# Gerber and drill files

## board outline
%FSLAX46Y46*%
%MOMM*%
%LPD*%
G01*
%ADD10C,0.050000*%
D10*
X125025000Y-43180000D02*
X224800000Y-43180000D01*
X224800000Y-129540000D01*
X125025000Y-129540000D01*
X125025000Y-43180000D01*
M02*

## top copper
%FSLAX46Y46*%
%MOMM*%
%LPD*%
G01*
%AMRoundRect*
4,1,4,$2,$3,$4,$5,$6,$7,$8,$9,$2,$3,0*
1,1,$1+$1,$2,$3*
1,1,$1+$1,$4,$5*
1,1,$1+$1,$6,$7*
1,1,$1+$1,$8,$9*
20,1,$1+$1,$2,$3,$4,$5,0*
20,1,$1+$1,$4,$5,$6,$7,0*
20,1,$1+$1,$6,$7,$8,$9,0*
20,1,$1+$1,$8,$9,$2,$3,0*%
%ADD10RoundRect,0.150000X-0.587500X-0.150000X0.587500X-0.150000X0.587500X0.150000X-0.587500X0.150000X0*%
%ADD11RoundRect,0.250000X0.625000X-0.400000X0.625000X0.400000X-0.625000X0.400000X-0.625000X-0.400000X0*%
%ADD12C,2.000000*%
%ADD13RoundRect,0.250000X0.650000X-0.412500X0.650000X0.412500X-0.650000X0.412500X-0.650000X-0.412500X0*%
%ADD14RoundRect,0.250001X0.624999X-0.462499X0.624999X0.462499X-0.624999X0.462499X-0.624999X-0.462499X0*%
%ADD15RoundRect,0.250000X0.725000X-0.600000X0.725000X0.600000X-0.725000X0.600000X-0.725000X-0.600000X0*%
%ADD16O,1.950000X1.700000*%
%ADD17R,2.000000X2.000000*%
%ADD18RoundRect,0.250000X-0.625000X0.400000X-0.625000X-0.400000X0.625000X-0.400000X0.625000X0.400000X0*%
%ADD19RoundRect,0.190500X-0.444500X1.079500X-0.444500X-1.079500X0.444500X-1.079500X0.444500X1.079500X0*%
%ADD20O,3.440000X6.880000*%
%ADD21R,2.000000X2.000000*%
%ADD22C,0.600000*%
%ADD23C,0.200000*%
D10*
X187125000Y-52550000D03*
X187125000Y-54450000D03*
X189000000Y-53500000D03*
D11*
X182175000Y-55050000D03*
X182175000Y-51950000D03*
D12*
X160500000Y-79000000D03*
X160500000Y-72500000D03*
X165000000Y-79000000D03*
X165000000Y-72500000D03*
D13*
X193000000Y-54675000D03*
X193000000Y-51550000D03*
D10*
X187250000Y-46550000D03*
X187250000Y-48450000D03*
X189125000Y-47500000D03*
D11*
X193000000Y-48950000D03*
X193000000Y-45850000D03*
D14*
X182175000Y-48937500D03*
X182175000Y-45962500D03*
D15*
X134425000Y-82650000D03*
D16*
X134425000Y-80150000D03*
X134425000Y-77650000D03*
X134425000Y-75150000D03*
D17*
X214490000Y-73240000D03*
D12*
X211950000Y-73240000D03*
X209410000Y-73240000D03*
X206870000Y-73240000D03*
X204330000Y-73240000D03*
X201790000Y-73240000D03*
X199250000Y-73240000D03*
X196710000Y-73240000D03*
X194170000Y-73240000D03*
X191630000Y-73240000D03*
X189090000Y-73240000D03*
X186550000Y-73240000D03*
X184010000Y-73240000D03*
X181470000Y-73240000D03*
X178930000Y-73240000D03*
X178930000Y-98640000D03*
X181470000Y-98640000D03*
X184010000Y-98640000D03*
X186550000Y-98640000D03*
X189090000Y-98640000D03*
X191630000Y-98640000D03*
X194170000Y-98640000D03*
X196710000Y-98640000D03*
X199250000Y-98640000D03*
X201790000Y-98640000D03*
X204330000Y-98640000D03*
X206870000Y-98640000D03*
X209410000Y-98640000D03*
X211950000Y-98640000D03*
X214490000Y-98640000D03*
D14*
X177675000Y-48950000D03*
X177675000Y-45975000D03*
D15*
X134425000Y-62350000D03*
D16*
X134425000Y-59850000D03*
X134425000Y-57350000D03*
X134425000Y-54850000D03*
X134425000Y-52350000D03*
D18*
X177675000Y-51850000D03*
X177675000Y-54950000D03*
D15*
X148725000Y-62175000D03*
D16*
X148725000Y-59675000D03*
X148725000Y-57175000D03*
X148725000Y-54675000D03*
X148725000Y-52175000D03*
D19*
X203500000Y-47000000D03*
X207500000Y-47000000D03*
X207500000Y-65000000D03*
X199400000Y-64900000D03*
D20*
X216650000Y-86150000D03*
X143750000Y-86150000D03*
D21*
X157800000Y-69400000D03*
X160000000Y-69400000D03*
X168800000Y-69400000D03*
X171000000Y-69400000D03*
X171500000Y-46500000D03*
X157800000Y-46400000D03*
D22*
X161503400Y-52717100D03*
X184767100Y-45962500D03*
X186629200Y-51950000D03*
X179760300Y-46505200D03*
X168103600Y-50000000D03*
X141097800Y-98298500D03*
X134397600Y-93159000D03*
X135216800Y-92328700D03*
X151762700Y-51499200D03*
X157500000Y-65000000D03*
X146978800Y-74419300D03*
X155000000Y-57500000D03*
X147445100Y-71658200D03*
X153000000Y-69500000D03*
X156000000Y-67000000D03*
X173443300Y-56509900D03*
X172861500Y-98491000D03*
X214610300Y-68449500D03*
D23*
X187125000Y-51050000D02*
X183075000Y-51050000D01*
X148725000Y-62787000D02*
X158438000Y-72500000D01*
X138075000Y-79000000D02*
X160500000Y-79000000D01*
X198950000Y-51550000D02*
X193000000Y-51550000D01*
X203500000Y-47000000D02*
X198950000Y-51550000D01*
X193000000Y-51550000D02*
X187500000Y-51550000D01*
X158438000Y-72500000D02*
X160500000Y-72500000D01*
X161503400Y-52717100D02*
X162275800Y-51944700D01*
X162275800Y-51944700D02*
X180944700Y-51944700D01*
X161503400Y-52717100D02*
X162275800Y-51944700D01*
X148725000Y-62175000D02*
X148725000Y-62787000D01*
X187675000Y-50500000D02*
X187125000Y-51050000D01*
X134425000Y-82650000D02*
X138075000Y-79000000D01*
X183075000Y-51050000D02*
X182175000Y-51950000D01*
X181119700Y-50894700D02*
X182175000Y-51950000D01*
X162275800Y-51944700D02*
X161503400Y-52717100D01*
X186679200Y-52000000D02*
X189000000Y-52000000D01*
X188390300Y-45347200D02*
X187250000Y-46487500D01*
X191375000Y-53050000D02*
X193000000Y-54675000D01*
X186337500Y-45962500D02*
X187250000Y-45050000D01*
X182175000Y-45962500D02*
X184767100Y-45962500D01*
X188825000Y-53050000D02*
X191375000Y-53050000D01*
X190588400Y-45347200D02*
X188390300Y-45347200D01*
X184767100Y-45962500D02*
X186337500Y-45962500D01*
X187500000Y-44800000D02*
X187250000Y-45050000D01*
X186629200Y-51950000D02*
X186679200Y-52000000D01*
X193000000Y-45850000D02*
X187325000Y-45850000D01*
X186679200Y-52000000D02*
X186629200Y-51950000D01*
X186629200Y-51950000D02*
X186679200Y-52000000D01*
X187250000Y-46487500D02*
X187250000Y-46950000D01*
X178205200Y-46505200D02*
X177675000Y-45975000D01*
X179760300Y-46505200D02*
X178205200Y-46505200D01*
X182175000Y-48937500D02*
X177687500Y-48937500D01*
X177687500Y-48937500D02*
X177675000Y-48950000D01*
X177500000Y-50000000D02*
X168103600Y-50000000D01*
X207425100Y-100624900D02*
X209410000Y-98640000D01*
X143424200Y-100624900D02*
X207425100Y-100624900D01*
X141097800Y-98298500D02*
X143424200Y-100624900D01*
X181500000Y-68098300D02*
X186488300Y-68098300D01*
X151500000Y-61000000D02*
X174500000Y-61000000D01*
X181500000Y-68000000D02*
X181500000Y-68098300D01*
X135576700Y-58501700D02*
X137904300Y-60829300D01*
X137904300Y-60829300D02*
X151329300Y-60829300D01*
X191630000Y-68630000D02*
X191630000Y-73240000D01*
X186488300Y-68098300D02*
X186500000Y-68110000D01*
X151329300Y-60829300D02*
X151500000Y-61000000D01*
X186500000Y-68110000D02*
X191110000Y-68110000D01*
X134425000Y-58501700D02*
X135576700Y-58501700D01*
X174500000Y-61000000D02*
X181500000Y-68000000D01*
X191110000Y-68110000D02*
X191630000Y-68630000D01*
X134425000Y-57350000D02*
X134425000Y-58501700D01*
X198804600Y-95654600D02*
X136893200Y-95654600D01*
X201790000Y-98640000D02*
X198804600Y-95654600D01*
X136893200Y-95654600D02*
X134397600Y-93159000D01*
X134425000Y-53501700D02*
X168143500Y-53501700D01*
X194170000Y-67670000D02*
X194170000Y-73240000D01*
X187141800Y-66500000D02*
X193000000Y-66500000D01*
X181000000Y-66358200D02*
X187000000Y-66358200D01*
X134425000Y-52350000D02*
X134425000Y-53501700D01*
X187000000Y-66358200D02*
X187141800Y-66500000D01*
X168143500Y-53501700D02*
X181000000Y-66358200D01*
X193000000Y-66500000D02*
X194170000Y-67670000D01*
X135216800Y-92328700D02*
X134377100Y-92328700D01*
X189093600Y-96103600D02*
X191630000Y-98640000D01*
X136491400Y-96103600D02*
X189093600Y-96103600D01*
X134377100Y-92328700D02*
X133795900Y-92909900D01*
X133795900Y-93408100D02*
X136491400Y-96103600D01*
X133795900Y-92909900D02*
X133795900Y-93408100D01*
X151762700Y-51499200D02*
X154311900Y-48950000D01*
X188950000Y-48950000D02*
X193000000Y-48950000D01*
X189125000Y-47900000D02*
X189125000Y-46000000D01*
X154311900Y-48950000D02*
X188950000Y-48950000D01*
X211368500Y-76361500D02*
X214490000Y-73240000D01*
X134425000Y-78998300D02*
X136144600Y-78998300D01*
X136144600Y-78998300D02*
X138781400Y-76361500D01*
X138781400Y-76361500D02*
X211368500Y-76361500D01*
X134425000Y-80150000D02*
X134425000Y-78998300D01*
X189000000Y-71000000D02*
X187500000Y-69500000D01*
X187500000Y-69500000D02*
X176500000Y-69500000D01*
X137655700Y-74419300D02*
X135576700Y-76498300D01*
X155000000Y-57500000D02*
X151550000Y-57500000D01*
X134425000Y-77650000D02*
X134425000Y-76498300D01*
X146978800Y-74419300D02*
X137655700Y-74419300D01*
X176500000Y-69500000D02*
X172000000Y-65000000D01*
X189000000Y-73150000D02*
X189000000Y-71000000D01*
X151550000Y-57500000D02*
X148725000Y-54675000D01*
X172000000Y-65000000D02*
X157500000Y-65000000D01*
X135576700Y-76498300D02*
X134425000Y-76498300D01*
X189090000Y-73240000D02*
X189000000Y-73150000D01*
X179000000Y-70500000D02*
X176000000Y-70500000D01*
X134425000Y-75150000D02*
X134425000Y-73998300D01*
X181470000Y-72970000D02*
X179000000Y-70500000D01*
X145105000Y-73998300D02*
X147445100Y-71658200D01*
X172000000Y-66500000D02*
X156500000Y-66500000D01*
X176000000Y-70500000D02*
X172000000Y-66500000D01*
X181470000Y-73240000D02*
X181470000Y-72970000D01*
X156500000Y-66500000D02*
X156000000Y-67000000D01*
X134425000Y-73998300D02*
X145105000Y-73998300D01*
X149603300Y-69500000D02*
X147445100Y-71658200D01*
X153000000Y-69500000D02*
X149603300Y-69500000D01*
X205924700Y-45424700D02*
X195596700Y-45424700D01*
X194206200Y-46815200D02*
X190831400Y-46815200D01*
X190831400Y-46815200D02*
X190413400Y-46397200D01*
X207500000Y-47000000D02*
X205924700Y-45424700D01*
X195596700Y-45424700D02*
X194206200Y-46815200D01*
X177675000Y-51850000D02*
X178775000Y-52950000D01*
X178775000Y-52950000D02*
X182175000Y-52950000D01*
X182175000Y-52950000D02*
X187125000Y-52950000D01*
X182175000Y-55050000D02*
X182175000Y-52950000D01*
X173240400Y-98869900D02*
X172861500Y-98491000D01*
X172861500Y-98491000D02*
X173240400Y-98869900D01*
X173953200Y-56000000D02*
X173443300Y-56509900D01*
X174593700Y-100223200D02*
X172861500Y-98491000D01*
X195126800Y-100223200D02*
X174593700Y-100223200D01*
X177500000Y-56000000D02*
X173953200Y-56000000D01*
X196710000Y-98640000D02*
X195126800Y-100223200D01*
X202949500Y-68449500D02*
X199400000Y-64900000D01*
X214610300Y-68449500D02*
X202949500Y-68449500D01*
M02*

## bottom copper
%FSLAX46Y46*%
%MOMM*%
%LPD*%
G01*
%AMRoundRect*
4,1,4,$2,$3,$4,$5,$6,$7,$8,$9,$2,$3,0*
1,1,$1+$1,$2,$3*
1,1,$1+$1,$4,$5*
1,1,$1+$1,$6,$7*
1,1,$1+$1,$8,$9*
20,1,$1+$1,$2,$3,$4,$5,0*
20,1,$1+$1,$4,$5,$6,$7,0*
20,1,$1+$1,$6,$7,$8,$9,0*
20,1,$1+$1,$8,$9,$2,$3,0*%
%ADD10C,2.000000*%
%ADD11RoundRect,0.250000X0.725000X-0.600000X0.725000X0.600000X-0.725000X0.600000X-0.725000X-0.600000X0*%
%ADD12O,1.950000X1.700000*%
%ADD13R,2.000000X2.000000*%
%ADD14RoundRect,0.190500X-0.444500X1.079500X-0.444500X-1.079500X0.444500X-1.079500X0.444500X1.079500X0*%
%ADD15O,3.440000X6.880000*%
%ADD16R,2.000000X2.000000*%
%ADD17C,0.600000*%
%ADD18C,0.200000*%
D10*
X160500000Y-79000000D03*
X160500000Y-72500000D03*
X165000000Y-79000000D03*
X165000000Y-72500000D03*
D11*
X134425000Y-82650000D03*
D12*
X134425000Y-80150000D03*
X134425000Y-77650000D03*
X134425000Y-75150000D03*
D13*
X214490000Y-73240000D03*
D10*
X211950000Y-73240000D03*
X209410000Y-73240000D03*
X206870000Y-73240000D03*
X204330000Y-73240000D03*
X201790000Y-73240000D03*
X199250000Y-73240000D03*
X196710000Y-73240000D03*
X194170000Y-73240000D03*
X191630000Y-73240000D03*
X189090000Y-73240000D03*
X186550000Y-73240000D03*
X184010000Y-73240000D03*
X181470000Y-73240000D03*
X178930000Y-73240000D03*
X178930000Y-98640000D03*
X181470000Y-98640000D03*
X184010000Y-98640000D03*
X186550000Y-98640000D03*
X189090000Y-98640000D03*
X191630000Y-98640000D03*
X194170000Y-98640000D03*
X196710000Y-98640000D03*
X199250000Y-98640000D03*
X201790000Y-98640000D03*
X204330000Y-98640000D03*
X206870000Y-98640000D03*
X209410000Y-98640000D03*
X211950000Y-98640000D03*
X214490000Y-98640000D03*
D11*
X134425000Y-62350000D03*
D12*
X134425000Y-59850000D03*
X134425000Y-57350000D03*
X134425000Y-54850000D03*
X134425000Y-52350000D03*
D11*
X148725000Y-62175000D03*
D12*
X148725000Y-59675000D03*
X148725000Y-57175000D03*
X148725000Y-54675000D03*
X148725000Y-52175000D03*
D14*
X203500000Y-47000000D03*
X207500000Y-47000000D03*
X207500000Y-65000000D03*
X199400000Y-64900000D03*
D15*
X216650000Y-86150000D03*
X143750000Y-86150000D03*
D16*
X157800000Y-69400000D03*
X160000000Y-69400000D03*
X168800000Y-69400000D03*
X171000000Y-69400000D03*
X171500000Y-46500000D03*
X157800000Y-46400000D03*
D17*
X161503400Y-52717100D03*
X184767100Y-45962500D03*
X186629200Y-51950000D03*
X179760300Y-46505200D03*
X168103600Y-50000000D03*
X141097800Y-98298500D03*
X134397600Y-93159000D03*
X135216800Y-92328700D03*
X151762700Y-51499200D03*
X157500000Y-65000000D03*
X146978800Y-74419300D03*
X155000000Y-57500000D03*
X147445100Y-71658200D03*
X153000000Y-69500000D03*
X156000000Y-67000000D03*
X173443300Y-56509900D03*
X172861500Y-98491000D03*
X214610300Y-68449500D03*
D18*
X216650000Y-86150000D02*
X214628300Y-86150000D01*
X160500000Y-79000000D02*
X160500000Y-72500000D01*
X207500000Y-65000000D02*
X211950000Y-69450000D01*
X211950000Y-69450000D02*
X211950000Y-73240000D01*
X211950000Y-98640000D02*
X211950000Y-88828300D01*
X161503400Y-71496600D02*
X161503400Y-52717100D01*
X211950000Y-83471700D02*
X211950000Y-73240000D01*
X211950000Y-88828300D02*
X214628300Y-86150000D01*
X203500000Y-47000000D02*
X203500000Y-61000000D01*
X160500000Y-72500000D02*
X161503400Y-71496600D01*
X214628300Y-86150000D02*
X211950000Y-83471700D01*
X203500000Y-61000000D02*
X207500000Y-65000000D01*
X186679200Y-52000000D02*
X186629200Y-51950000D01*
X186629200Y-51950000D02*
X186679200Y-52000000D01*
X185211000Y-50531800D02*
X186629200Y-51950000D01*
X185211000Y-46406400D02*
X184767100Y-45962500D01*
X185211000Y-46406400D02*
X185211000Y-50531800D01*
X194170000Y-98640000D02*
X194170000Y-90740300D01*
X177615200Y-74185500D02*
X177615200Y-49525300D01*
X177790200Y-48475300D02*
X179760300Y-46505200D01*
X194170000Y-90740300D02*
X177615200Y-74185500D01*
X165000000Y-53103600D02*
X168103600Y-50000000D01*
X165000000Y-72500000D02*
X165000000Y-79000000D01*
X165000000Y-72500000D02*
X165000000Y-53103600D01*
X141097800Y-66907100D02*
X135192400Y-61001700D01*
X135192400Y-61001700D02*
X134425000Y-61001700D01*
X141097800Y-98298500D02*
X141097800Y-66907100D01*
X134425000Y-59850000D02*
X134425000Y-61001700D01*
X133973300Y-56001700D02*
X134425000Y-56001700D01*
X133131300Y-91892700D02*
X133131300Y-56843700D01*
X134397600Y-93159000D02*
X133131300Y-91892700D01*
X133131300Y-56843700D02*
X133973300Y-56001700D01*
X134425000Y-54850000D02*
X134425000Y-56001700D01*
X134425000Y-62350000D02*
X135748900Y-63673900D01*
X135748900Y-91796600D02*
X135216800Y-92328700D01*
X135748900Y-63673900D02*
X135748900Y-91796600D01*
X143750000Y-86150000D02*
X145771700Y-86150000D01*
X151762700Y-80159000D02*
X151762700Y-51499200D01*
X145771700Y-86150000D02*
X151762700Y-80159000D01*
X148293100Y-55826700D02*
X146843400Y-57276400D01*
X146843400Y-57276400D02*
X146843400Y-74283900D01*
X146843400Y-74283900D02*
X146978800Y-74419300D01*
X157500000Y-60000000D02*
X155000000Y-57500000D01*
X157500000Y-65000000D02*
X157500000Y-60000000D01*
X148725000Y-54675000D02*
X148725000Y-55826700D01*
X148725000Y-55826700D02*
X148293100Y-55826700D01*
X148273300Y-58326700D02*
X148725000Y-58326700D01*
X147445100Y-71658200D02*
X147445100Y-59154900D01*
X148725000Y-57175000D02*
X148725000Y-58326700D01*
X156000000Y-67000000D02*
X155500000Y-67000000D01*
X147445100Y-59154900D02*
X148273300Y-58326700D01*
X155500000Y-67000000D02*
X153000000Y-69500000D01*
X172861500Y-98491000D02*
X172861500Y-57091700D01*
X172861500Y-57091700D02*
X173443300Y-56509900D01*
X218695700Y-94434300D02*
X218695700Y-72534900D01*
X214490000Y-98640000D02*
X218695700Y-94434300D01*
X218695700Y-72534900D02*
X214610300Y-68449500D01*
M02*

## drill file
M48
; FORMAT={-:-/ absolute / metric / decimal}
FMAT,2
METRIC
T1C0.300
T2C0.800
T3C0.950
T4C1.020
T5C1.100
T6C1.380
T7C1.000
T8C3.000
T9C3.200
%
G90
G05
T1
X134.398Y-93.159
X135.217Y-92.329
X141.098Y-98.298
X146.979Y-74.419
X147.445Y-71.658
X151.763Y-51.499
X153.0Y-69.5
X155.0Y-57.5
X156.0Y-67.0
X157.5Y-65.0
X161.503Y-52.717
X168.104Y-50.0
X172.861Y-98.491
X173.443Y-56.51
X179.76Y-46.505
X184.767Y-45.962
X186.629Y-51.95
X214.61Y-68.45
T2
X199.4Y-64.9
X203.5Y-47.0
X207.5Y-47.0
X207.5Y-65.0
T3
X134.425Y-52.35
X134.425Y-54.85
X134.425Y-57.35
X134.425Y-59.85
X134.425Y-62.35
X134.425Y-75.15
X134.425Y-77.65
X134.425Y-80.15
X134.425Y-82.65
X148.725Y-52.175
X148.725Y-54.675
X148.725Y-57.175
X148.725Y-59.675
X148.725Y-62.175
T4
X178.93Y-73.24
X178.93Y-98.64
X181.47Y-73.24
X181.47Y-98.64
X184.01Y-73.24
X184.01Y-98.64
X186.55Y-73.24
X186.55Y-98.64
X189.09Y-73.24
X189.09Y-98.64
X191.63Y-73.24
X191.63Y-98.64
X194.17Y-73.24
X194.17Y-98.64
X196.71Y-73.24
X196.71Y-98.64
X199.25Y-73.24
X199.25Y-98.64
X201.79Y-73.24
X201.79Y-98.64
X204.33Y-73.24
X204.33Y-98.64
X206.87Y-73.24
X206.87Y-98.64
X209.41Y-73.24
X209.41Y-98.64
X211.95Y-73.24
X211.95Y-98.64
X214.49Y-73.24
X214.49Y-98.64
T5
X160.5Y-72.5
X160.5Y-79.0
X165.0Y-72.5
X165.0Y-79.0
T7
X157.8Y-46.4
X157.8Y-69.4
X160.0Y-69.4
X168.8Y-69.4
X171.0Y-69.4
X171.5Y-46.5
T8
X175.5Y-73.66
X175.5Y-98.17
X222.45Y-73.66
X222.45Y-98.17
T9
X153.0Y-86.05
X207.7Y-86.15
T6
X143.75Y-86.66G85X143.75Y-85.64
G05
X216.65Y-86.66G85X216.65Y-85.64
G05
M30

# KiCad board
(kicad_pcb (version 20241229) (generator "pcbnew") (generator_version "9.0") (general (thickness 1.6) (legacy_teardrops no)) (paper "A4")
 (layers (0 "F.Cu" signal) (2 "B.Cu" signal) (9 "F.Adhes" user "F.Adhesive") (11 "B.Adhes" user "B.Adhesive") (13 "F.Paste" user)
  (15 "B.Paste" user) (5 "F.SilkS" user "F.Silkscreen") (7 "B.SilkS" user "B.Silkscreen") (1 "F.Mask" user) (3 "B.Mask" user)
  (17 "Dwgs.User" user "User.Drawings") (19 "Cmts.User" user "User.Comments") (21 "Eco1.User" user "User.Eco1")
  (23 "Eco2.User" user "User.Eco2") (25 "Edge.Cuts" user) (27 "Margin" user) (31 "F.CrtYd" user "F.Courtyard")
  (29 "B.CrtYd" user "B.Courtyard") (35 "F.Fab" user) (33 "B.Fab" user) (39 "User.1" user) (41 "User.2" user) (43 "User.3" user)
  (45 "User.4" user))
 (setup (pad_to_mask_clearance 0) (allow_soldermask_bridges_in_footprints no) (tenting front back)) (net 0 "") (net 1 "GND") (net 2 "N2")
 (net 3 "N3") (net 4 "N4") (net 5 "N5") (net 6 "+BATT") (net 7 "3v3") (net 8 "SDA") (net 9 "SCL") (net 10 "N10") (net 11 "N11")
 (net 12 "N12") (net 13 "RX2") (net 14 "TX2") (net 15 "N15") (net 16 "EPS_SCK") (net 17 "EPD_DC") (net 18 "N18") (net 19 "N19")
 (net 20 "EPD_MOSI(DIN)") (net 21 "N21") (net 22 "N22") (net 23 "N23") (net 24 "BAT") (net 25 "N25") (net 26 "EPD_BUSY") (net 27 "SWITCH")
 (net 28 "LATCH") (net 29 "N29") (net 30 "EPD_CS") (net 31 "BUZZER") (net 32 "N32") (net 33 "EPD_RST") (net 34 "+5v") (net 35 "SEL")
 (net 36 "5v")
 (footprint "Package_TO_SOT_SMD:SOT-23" (layer "F.Cu") (at 188.0625 53.5)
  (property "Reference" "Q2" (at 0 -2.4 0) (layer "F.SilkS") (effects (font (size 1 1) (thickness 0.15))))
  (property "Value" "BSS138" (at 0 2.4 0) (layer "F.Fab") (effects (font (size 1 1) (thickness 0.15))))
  (pad "1" smd roundrect (at -0.9375 -0.95) (size 1.475 0.6) (layers "F.Cu" "F.Mask" "F.Paste") (roundrect_rratio 0.25) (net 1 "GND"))
  (pad "2" smd roundrect (at -0.9375 0.95) (size 1.475 0.6) (layers "F.Cu" "F.Mask" "F.Paste") (roundrect_rratio 0.25) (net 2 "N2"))
  (pad "3" smd roundrect (at 0.9375 0) (size 1.475 0.6) (layers "F.Cu" "F.Mask" "F.Paste") (roundrect_rratio 0.25) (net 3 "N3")))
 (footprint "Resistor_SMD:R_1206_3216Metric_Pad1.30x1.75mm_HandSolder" (layer "F.Cu") (at 182.175 53.5 90)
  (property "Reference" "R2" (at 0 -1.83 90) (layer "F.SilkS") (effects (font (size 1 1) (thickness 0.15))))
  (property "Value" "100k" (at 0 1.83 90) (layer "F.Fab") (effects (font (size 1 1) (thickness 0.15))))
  (pad "1" smd roundrect (at -1.55 0 90) (size 1.3 1.75) (layers "F.Cu" "F.Mask" "F.Paste") (roundrect_rratio 0.192308) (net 2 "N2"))
  (pad "2" smd roundrect (at 1.55 0 90) (size 1.3 1.75) (layers "F.Cu" "F.Mask" "F.Paste") (roundrect_rratio 0.192308) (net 1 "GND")))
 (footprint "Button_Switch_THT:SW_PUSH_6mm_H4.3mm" (layer "F.Cu") (at 160.5 79 90)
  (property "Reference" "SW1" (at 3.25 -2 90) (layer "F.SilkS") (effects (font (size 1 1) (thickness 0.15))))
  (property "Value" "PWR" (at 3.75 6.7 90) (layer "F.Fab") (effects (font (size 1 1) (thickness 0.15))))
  (pad "1" thru_hole circle (at 0 0 180) (size 2 2) (drill 1.1) (layers "*.Cu" "*.Mask") (remove_unused_layers no) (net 1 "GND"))
  (pad "1" thru_hole circle (at 6.5 0 180) (size 2 2) (drill 1.1) (layers "*.Cu" "*.Mask") (remove_unused_layers no) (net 1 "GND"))
  (pad "2" thru_hole circle (at 0 4.5 180) (size 2 2) (drill 1.1) (layers "*.Cu" "*.Mask") (remove_unused_layers no) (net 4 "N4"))
  (pad "2" thru_hole circle (at 6.5 4.5 180) (size 2 2) (drill 1.1) (layers "*.Cu" "*.Mask") (remove_unused_layers no) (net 4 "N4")))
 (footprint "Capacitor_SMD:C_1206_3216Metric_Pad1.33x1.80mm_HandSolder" (layer "F.Cu") (at 193 53.1125 90)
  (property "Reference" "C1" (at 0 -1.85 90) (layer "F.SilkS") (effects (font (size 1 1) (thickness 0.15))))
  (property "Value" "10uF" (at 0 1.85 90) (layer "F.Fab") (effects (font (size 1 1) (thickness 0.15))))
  (pad "1" smd roundrect (at -1.5625 0 90) (size 1.325 1.8) (layers "F.Cu" "F.Mask" "F.Paste") (roundrect_rratio 0.188679) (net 3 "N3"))
  (pad "2" smd roundrect (at 1.5625 0 90) (size 1.325 1.8) (layers "F.Cu" "F.Mask" "F.Paste") (roundrect_rratio 0.188679) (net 1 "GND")))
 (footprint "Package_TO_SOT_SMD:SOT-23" (layer "F.Cu") (at 188.1875 47.5)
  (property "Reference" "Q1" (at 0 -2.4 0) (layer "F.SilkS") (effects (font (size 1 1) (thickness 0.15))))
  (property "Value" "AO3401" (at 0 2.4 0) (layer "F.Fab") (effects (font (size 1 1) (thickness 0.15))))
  (pad "1" smd roundrect (at -0.9375 -0.95) (size 1.475 0.6) (layers "F.Cu" "F.Mask" "F.Paste") (roundrect_rratio 0.25) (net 3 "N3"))
  (pad "2" smd roundrect (at -0.9375 0.95) (size 1.475 0.6) (layers "F.Cu" "F.Mask" "F.Paste") (roundrect_rratio 0.25) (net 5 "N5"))
  (pad "3" smd roundrect (at 0.9375 0) (size 1.475 0.6) (layers "F.Cu" "F.Mask" "F.Paste") (roundrect_rratio 0.25) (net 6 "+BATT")))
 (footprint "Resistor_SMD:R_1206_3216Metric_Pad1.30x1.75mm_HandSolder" (layer "F.Cu") (at 193 47.4 90)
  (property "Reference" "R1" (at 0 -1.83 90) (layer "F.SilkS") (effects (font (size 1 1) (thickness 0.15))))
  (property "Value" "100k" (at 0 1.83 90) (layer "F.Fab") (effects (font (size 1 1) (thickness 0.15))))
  (pad "1" smd roundrect (at -1.55 0 90) (size 1.3 1.75) (layers "F.Cu" "F.Mask" "F.Paste") (roundrect_rratio 0.192308) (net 6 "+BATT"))
  (pad "2" smd roundrect (at 1.55 0 90) (size 1.3 1.75) (layers "F.Cu" "F.Mask" "F.Paste") (roundrect_rratio 0.192308) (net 3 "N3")))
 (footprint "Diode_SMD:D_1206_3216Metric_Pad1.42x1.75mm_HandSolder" (layer "F.Cu") (at 182.175 47.45 90)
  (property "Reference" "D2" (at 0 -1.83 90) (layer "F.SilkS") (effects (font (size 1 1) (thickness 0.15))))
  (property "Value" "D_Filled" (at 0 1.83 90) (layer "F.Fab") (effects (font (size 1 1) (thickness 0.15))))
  (pad "1" smd roundrect (at -1.4875 0 90) (size 1.425 1.75) (layers "F.Cu" "F.Mask" "F.Paste") (roundrect_rratio 0.175439) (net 4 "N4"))
  (pad "2" smd roundrect (at 1.4875 0 90) (size 1.425 1.75) (layers "F.Cu" "F.Mask" "F.Paste") (roundrect_rratio 0.175439) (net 3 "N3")))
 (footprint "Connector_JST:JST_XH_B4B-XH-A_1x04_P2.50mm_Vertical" (layer "F.Cu") (at 134.425 82.65 90)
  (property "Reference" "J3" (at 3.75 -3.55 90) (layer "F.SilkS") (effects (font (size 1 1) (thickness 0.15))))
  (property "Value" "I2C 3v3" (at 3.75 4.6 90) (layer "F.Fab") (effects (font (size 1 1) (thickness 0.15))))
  (pad "1" thru_hole roundrect (at 0 0 90) (size 1.7 1.95) (drill 0.95) (layers "*.Cu" "*.Mask") (remove_unused_layers no)
   (roundrect_rratio 0.147059) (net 1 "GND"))
  (pad "2" thru_hole oval (at 2.5 0 90) (size 1.7 1.95) (drill 0.95) (layers "*.Cu" "*.Mask") (remove_unused_layers no) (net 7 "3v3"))
  (pad "3" thru_hole oval (at 5 0 90) (size 1.7 1.95) (drill 0.95) (layers "*.Cu" "*.Mask") (remove_unused_layers no) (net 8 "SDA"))
  (pad "4" thru_hole oval (at 7.5 0 90) (size 1.7 1.95) (drill 0.95) (layers "*.Cu" "*.Mask") (remove_unused_layers no) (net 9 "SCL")))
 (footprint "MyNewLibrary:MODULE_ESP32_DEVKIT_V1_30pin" (layer "F.Cu") (at 198.975 85.94 -90)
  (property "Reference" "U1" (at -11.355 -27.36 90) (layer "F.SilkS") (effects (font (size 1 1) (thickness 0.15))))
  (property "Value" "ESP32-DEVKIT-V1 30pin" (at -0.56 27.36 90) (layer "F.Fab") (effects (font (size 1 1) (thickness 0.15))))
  (pad "" np_thru_hole circle (at -12.28 -23.475 270) (size 3 3) (drill 3) (layers "*.Cu" "*.Mask"))
  (pad "" np_thru_hole circle (at -12.28 23.475 270) (size 3 3) (drill 3) (layers "*.Cu" "*.Mask"))
  (pad "" np_thru_hole circle (at 12.23 -23.475 270) (size 3 3) (drill 3) (layers "*.Cu" "*.Mask"))
  (pad "" np_thru_hole circle (at 12.23 23.475 270) (size 3 3) (drill 3) (layers "*.Cu" "*.Mask"))
  (pad "1" thru_hole rect (at -12.7 -15.515 270) (size 2 2) (drill 1.02) (layers "*.Cu" "*.Mask") (remove_unused_layers no) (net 7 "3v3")
   (solder_mask_margin 0.102))
  (pad "2" thru_hole circle (at -12.7 -12.975 270) (size 2 2) (drill 1.02) (layers "*.Cu" "*.Mask") (remove_unused_layers no) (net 1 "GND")
   (solder_mask_margin 0.102))
  (pad "3" thru_hole circle (at -12.7 -10.435 270) (size 2 2) (drill 1.02) (layers "*.Cu" "*.Mask") (remove_unused_layers no) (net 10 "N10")
   (solder_mask_margin 0.102))
  (pad "4" thru_hole circle (at -12.7 -7.895 270) (size 2 2) (drill 1.02) (layers "*.Cu" "*.Mask") (remove_unused_layers no) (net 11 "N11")
   (solder_mask_margin 0.102))
  (pad "5" thru_hole circle (at -12.7 -5.355 270) (size 2 2) (drill 1.02) (layers "*.Cu" "*.Mask") (remove_unused_layers no) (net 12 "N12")
   (solder_mask_margin 0.102))
  (pad "6" thru_hole circle (at -12.7 -2.815 270) (size 2 2) (drill 1.02) (layers "*.Cu" "*.Mask") (remove_unused_layers no) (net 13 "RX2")
   (solder_mask_margin 0.102))
  (pad "7" thru_hole circle (at -12.7 -0.275 270) (size 2 2) (drill 1.02) (layers "*.Cu" "*.Mask") (remove_unused_layers no) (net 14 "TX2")
   (solder_mask_margin 0.102))
  (pad "8" thru_hole circle (at -12.7 2.265 270) (size 2 2) (drill 1.02) (layers "*.Cu" "*.Mask") (remove_unused_layers no) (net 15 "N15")
   (solder_mask_margin 0.102))
  (pad "9" thru_hole circle (at -12.7 4.805 270) (size 2 2) (drill 1.02) (layers "*.Cu" "*.Mask") (remove_unused_layers no)
   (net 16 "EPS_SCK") (solder_mask_margin 0.102))
  (pad "10" thru_hole circle (at -12.7 7.345 270) (size 2 2) (drill 1.02) (layers "*.Cu" "*.Mask") (remove_unused_layers no)
   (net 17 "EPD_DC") (solder_mask_margin 0.102))
  (pad "11" thru_hole circle (at -12.7 9.885 270) (size 2 2) (drill 1.02) (layers "*.Cu" "*.Mask") (remove_unused_layers no) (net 8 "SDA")
   (solder_mask_margin 0.102))
  (pad "12" thru_hole circle (at -12.7 12.425 270) (size 2 2) (drill 1.02) (layers "*.Cu" "*.Mask") (remove_unused_layers no) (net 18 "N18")
   (solder_mask_margin 0.102))
  (pad "13" thru_hole circle (at -12.7 14.965 270) (size 2 2) (drill 1.02) (layers "*.Cu" "*.Mask") (remove_unused_layers no) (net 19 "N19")
   (solder_mask_margin 0.102))
  (pad "14" thru_hole circle (at -12.7 17.505 270) (size 2 2) (drill 1.02) (layers "*.Cu" "*.Mask") (remove_unused_layers no) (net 9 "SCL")
   (solder_mask_margin 0.102))
  (pad "15" thru_hole circle (at -12.7 20.045 270) (size 2 2) (drill 1.02) (layers "*.Cu" "*.Mask") (remove_unused_layers no)
   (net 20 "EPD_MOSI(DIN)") (solder_mask_margin 0.102))
  (pad "16" thru_hole circle (at 12.7 20.045 270) (size 2 2) (drill 1.02) (layers "*.Cu" "*.Mask") (remove_unused_layers no) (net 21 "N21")
   (solder_mask_margin 0.102))
  (pad "17" thru_hole circle (at 12.7 17.505 270) (size 2 2) (drill 1.02) (layers "*.Cu" "*.Mask") (remove_unused_layers no) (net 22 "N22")
   (solder_mask_margin 0.102))
  (pad "18" thru_hole circle (at 12.7 14.965 270) (size 2 2) (drill 1.02) (layers "*.Cu" "*.Mask") (remove_unused_layers no) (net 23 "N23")
   (solder_mask_margin 0.102))
  (pad "19" thru_hole circle (at 12.7 12.425 270) (size 2 2) (drill 1.02) (layers "*.Cu" "*.Mask") (remove_unused_layers no) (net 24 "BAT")
   (solder_mask_margin 0.102))
  (pad "20" thru_hole circle (at 12.7 9.885 270) (size 2 2) (drill 1.02) (layers "*.Cu" "*.Mask") (remove_unused_layers no) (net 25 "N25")
   (solder_mask_margin 0.102))
  (pad "21" thru_hole circle (at 12.7 7.345 270) (size 2 2) (drill 1.02) (layers "*.Cu" "*.Mask") (remove_unused_layers no)
   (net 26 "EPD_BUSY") (solder_mask_margin 0.102))
  (pad "22" thru_hole circle (at 12.7 4.805 270) (size 2 2) (drill 1.02) (layers "*.Cu" "*.Mask") (remove_unused_layers no)
   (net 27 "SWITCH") (solder_mask_margin 0.102))
  (pad "23" thru_hole circle (at 12.7 2.265 270) (size 2 2) (drill 1.02) (layers "*.Cu" "*.Mask") (remove_unused_layers no) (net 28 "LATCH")
   (solder_mask_margin 0.102))
  (pad "24" thru_hole circle (at 12.7 -0.275 270) (size 2 2) (drill 1.02) (layers "*.Cu" "*.Mask") (remove_unused_layers no) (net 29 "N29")
   (solder_mask_margin 0.102))
  (pad "25" thru_hole circle (at 12.7 -2.815 270) (size 2 2) (drill 1.02) (layers "*.Cu" "*.Mask") (remove_unused_layers no)
   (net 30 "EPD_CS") (solder_mask_margin 0.102))
  (pad "26" thru_hole circle (at 12.7 -5.355 270) (size 2 2) (drill 1.02) (layers "*.Cu" "*.Mask") (remove_unused_layers no)
   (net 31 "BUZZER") (solder_mask_margin 0.102))
  (pad "27" thru_hole circle (at 12.7 -7.895 270) (size 2 2) (drill 1.02) (layers "*.Cu" "*.Mask") (remove_unused_layers no) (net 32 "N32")
   (solder_mask_margin 0.102))
  (pad "28" thru_hole circle (at 12.7 -10.435 270) (size 2 2) (drill 1.02) (layers "*.Cu" "*.Mask") (remove_unused_layers no)
   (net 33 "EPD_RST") (solder_mask_margin 0.102))
  (pad "29" thru_hole circle (at 12.7 -12.975 270) (size 2 2) (drill 1.02) (layers "*.Cu" "*.Mask") (remove_unused_layers no) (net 1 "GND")
   (solder_mask_margin 0.102))
  (pad "30" thru_hole circle (at 12.7 -15.515 270) (size 2 2) (drill 1.02) (layers "*.Cu" "*.Mask") (remove_unused_layers no) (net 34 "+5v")
   (solder_mask_margin 0.102))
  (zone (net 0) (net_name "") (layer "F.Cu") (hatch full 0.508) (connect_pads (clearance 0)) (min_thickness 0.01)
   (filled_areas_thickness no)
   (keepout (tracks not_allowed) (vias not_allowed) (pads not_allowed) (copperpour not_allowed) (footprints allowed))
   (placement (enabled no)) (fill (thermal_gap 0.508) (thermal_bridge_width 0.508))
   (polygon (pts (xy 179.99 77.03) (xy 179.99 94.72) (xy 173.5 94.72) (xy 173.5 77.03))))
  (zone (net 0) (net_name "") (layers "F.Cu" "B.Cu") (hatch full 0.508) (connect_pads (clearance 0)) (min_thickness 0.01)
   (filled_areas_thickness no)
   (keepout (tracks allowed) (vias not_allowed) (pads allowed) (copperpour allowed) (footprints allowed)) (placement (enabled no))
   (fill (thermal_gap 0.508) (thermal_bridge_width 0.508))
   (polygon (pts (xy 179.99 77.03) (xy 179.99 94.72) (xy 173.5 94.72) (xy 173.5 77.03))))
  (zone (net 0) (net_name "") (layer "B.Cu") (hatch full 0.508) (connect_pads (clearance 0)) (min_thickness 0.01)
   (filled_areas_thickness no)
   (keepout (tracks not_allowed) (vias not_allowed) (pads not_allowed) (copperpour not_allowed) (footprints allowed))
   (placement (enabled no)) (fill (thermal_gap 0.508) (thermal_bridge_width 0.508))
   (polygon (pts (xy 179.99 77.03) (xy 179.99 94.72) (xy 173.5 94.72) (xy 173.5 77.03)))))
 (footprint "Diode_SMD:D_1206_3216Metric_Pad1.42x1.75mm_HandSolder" (layer "F.Cu") (at 177.675 47.4625 90)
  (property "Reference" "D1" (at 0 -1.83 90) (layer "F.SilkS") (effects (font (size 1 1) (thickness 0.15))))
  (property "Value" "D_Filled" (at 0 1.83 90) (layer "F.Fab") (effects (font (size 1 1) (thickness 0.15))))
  (pad "1" smd roundrect (at -1.4875 0 90) (size 1.425 1.75) (layers "F.Cu" "F.Mask" "F.Paste") (roundrect_rratio 0.175439) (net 4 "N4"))
  (pad "2" smd roundrect (at 1.4875 0 90) (size 1.425 1.75) (layers "F.Cu" "F.Mask" "F.Paste") (roundrect_rratio 0.175439) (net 27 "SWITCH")))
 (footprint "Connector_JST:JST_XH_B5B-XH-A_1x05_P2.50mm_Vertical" (layer "F.Cu") (at 134.425 62.35 90)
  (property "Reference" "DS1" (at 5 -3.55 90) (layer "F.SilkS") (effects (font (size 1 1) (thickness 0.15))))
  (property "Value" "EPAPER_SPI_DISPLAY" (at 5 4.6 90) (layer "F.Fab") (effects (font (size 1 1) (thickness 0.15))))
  (pad "1" thru_hole roundrect (at 0 0 90) (size 1.7 1.95) (drill 0.95) (layers "*.Cu" "*.Mask") (remove_unused_layers no)
   (roundrect_rratio 0.147059) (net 26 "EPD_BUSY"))
  (pad "2" thru_hole oval (at 2.5 0 90) (size 1.7 1.95) (drill 0.95) (layers "*.Cu" "*.Mask") (remove_unused_layers no) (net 33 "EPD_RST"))
  (pad "3" thru_hole oval (at 5 0 90) (size 1.7 1.95) (drill 0.95) (layers "*.Cu" "*.Mask") (remove_unused_layers no) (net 17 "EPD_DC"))
  (pad "4" thru_hole oval (at 7.5 0 90) (size 1.7 1.95) (drill 0.95) (layers "*.Cu" "*.Mask") (remove_unused_layers no) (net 30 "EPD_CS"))
  (pad "5" thru_hole oval (at 10 0 90) (size 1.7 1.95) (drill 0.95) (layers "*.Cu" "*.Mask") (remove_unused_layers no) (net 16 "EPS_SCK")))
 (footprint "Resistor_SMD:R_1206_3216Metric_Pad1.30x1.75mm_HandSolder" (layer "F.Cu") (at 177.675 53.4 -90)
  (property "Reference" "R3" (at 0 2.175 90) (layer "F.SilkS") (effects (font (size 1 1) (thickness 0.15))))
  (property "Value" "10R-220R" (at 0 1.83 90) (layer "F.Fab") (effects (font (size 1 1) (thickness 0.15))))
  (pad "1" smd roundrect (at -1.55 0 270) (size 1.3 1.75) (layers "F.Cu" "F.Mask" "F.Paste") (roundrect_rratio 0.192308) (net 2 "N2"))
  (pad "2" smd roundrect (at 1.55 0 270) (size 1.3 1.75) (layers "F.Cu" "F.Mask" "F.Paste") (roundrect_rratio 0.192308) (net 28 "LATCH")))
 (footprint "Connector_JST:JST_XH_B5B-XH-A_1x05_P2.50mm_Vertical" (layer "F.Cu") (at 148.725 62.175 90)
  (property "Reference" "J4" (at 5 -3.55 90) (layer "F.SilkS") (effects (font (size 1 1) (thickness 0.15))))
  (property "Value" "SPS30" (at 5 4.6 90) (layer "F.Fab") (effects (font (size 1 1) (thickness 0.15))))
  (pad "1" thru_hole roundrect (at 0 0 90) (size 1.7 1.95) (drill 0.95) (layers "*.Cu" "*.Mask") (remove_unused_layers no)
   (roundrect_rratio 0.147059) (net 1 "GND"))
  (pad "2" thru_hole oval (at 2.5 0 90) (size 1.7 1.95) (drill 0.95) (layers "*.Cu" "*.Mask") (remove_unused_layers no) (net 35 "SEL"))
  (pad "3" thru_hole oval (at 5 0 90) (size 1.7 1.95) (drill 0.95) (layers "*.Cu" "*.Mask") (remove_unused_layers no) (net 9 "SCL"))
  (pad "4" thru_hole oval (at 7.5 0 90) (size 1.7 1.95) (drill 0.95) (layers "*.Cu" "*.Mask") (remove_unused_layers no) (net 8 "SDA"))
  (pad "5" thru_hole oval (at 10 0 90) (size 1.7 1.95) (drill 0.95) (layers "*.Cu" "*.Mask") (remove_unused_layers no) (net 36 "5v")))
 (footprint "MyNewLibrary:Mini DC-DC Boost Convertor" (layer "B.Cu") (at 203.4 56.1 -90)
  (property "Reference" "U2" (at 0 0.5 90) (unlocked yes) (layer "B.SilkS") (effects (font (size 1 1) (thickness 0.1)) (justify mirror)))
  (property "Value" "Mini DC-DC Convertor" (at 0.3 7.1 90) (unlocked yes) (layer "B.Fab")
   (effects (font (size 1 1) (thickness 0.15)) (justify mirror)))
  (pad "1" thru_hole roundrect (at -9.1 -0.1 270) (size 2.54 1.27) (drill 0.8) (layers "*.Cu" "*.Mask") (remove_unused_layers no)
   (roundrect_rratio 0.15) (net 1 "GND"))
  (pad "2" thru_hole roundrect (at -9.1 -4.1 270) (size 2.54 1.27) (drill 0.8) (layers "*.Cu" "*.Mask") (remove_unused_layers no)
   (roundrect_rratio 0.15) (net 5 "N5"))
  (pad "3" thru_hole roundrect (at 8.9 -4.1 270) (size 2.54 1.27) (drill 0.8) (layers "*.Cu" "*.Mask") (remove_unused_layers no)
   (roundrect_rratio 0.15) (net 1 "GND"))
  (pad "4" thru_hole roundrect (at 8.8 4 270) (size 2.54 1.27) (drill 0.8) (layers "*.Cu" "*.Mask") (remove_unused_layers no)
   (roundrect_rratio 0.15) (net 34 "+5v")))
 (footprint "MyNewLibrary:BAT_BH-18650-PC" (layer "B.Cu") (at 180.2 86.15 180)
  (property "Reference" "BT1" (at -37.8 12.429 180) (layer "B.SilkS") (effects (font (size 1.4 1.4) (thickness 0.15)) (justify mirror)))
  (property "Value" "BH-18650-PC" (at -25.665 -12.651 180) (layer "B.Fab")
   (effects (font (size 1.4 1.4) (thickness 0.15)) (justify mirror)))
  (pad "" np_thru_hole circle (at -27.5 0 180) (size 3.2 3.2) (drill 3.2) (layers "*.Cu" "*.Mask"))
  (pad "" np_thru_hole circle (at 27.2 0.1 180) (size 3.2 3.2) (drill 3.2) (layers "*.Cu" "*.Mask"))
  (pad "N" thru_hole oval (at -36.45 0 180) (size 3.44 6.88) (drill oval 1.38 2.4) (layers "*.Cu" "*.Mask") (remove_unused_layers no)
   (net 1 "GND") (solder_mask_margin 0.102))
  (pad "P" thru_hole oval (at 36.45 0 180) (size 3.44 6.88) (drill oval 1.38 2.4) (layers "*.Cu" "*.Mask") (remove_unused_layers no)
   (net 6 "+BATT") (solder_mask_margin 0.102)))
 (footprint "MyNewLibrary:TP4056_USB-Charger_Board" (layer "B.Cu") (at 164.3 57 90)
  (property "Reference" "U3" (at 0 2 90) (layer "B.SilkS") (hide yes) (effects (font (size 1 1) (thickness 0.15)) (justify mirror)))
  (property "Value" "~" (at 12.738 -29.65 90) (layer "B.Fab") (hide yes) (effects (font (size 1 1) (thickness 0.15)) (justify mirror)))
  (pad "" np_thru_hole rect (at -12.4 -6.5 90) (size 2 2) (drill 1) (layers "*.Cu" "*.Mask"))
  (pad "" np_thru_hole rect (at -12.4 -4.3 90) (size 2 2) (drill 1) (layers "*.Cu" "*.Mask"))
  (pad "" np_thru_hole rect (at -12.4 4.5 90) (size 2 2) (drill 1) (layers "*.Cu" "*.Mask"))
  (pad "" np_thru_hole rect (at -12.4 6.7 90) (size 2 2) (drill 1) (layers "*.Cu" "*.Mask"))
  (pad "" np_thru_hole rect (at 10.5 7.2 90) (size 2 2) (drill 1) (layers "*.Cu" "*.Mask"))
  (pad "" np_thru_hole rect (at 10.6 -6.5 90) (size 2 2) (drill 1) (layers "*.Cu" "*.Mask")))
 (gr_rect (start 125.025 43.18) (end 224.8 129.54) (stroke (width 0.05) (type default)) (fill no) (layer "Edge.Cuts"))
 (segment (start 187.125 51.05) (end 183.075 51.05) (width 0.2) (layer "F.Cu") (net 1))
 (segment (start 148.725 62.787) (end 158.438 72.5) (width 0.2) (layer "F.Cu") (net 1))
 (segment (start 138.075 79) (end 160.5 79) (width 0.2) (layer "F.Cu") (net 1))
 (segment (start 198.95 51.55) (end 193 51.55) (width 0.2) (layer "F.Cu") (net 1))
 (segment (start 203.5 47) (end 198.95 51.55) (width 0.2) (layer "F.Cu") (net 1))
 (segment (start 193 51.55) (end 187.5 51.55) (width 0.2) (layer "F.Cu") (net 1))
 (segment (start 158.438 72.5) (end 160.5 72.5) (width 0.2) (layer "F.Cu") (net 1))
 (segment (start 161.5034 52.7171) (end 162.2758 51.9447) (width 0.2) (layer "F.Cu") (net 1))
 (segment (start 162.2758 51.9447) (end 180.9447 51.9447) (width 0.2) (layer "F.Cu") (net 1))
 (segment (start 161.5034 52.7171) (end 162.2758 51.9447) (width 0.2) (layer "F.Cu") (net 1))
 (segment (start 148.725 62.175) (end 148.725 62.787) (width 0.2) (layer "F.Cu") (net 1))
 (segment (start 187.675 50.5) (end 187.125 51.05) (width 0.2) (layer "F.Cu") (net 1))
 (segment (start 134.425 82.65) (end 138.075 79) (width 0.2) (layer "F.Cu") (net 1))
 (segment (start 183.075 51.05) (end 182.175 51.95) (width 0.2) (layer "F.Cu") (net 1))
 (segment (start 181.1197 50.8947) (end 182.175 51.95) (width 0.2) (layer "F.Cu") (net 1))
 (segment (start 162.2758 51.9447) (end 161.5034 52.7171) (width 0.2) (layer "F.Cu") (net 1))
 (via (at 161.5034 52.7171) (size 0.6) (drill 0.3) (layers "F.Cu" "B.Cu") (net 1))
 (segment (start 216.65 86.15) (end 214.6283 86.15) (width 0.2) (layer "B.Cu") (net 1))
 (segment (start 160.5 79) (end 160.5 72.5) (width 0.2) (layer "B.Cu") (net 1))
 (segment (start 207.5 65) (end 211.95 69.45) (width 0.2) (layer "B.Cu") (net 1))
 (segment (start 211.95 69.45) (end 211.95 73.24) (width 0.2) (layer "B.Cu") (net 1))
 (segment (start 211.95 98.64) (end 211.95 88.8283) (width 0.2) (layer "B.Cu") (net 1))
 (segment (start 161.5034 71.4966) (end 161.5034 52.7171) (width 0.2) (layer "B.Cu") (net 1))
 (segment (start 211.95 83.4717) (end 211.95 73.24) (width 0.2) (layer "B.Cu") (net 1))
 (segment (start 211.95 88.8283) (end 214.6283 86.15) (width 0.2) (layer "B.Cu") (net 1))
 (segment (start 203.5 47) (end 203.5 61) (width 0.2) (layer "B.Cu") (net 1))
 (segment (start 160.5 72.5) (end 161.5034 71.4966) (width 0.2) (layer "B.Cu") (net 1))
 (segment (start 214.6283 86.15) (end 211.95 83.4717) (width 0.2) (layer "B.Cu") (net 1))
 (segment (start 203.5 61) (end 207.5 65) (width 0.2) (layer "B.Cu") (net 1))
 (segment (start 186.6792 52) (end 189 52) (width 0.2) (layer "F.Cu") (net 3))
 (segment (start 188.3903 45.3472) (end 187.25 46.4875) (width 0.2) (layer "F.Cu") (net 3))
 (segment (start 191.375 53.05) (end 193 54.675) (width 0.2) (layer "F.Cu") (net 3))
 (segment (start 186.3375 45.9625) (end 187.25 45.05) (width 0.2) (layer "F.Cu") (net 3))
 (segment (start 182.175 45.9625) (end 184.7671 45.9625) (width 0.2) (layer "F.Cu") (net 3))
 (segment (start 188.825 53.05) (end 191.375 53.05) (width 0.2) (layer "F.Cu") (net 3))
 (segment (start 190.5884 45.3472) (end 188.3903 45.3472) (width 0.2) (layer "F.Cu") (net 3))
 (segment (start 184.7671 45.9625) (end 186.3375 45.9625) (width 0.2) (layer "F.Cu") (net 3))
 (segment (start 187.5 44.8) (end 187.25 45.05) (width 0.2) (layer "F.Cu") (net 3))
 (segment (start 186.6292 51.95) (end 186.6792 52) (width 0.2) (layer "F.Cu") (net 3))
 (segment (start 193 45.85) (end 187.325 45.85) (width 0.2) (layer "F.Cu") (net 3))
 (segment (start 186.6792 52) (end 186.6292 51.95) (width 0.2) (layer "F.Cu") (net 3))
 (segment (start 186.6292 51.95) (end 186.6792 52) (width 0.2) (layer "F.Cu") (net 3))
 (segment (start 187.25 46.4875) (end 187.25 46.95) (width 0.2) (layer "F.Cu") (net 3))
 (via (at 184.7671 45.9625) (size 0.6) (drill 0.3) (layers "F.Cu" "B.Cu") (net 3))
 (via (at 186.6292 51.95) (size 0.6) (drill 0.3) (layers "F.Cu" "B.Cu") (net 3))
 (segment (start 186.6792 52) (end 186.6292 51.95) (width 0.2) (layer "B.Cu") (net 3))
 (segment (start 186.6292 51.95) (end 186.6792 52) (width 0.2) (layer "B.Cu") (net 3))
 (segment (start 185.211 50.5318) (end 186.6292 51.95) (width 0.2) (layer "B.Cu") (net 3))
 (segment (start 185.211 46.4064) (end 184.7671 45.9625) (width 0.2) (layer "B.Cu") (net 3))
 (segment (start 185.211 46.4064) (end 185.211 50.5318) (width 0.2) (layer "B.Cu") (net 3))
 (segment (start 178.2052 46.5052) (end 177.675 45.975) (width 0.2) (layer "F.Cu") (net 27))
 (segment (start 179.7603 46.5052) (end 178.2052 46.5052) (width 0.2) (layer "F.Cu") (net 27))
 (via (at 179.7603 46.5052) (size 0.6) (drill 0.3) (layers "F.Cu" "B.Cu") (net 27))
 (segment (start 194.17 98.64) (end 194.17 90.7403) (width 0.2) (layer "B.Cu") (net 27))
 (segment (start 177.6152 74.1855) (end 177.6152 49.5253) (width 0.2) (layer "B.Cu") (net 27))
 (segment (start 177.7902 48.4753) (end 179.7603 46.5052) (width 0.2) (layer "B.Cu") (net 27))
 (segment (start 194.17 90.7403) (end 177.6152 74.1855) (width 0.2) (layer "B.Cu") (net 27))
 (segment (start 182.175 48.9375) (end 177.6875 48.9375) (width 0.2) (layer "F.Cu") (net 4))
 (segment (start 177.6875 48.9375) (end 177.675 48.95) (width 0.2) (layer "F.Cu") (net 4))
 (segment (start 177.5 50) (end 168.1036 50) (width 0.2) (layer "F.Cu") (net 4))
 (via (at 168.1036 50) (size 0.6) (drill 0.3) (layers "F.Cu" "B.Cu") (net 4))
 (segment (start 165 53.1036) (end 168.1036 50) (width 0.2) (layer "B.Cu") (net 4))
 (segment (start 165 72.5) (end 165 79) (width 0.2) (layer "B.Cu") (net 4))
 (segment (start 165 72.5) (end 165 53.1036) (width 0.2) (layer "B.Cu") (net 4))
 (segment (start 207.4251 100.6249) (end 209.41 98.64) (width 0.2) (layer "F.Cu") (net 33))
 (segment (start 143.4242 100.6249) (end 207.4251 100.6249) (width 0.2) (layer "F.Cu") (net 33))
 (segment (start 141.0978 98.2985) (end 143.4242 100.6249) (width 0.2) (layer "F.Cu") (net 33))
 (via (at 141.0978 98.2985) (size 0.6) (drill 0.3) (layers "F.Cu" "B.Cu") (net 33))
 (segment (start 141.0978 66.9071) (end 135.1924 61.0017) (width 0.2) (layer "B.Cu") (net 33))
 (segment (start 135.1924 61.0017) (end 134.425 61.0017) (width 0.2) (layer "B.Cu") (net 33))
 (segment (start 141.0978 98.2985) (end 141.0978 66.9071) (width 0.2) (layer "B.Cu") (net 33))
 (segment (start 134.425 59.85) (end 134.425 61.0017) (width 0.2) (layer "B.Cu") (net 33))
 (segment (start 181.5 68.0983) (end 186.4883 68.0983) (width 0.2) (layer "F.Cu") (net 17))
 (segment (start 151.5 61) (end 174.5 61) (width 0.2) (layer "F.Cu") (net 17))
 (segment (start 181.5 68) (end 181.5 68.0983) (width 0.2) (layer "F.Cu") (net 17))
 (segment (start 135.5767 58.5017) (end 137.9043 60.8293) (width 0.2) (layer "F.Cu") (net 17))
 (segment (start 137.9043 60.8293) (end 151.3293 60.8293) (width 0.2) (layer "F.Cu") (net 17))
 (segment (start 191.63 68.63) (end 191.63 73.24) (width 0.2) (layer "F.Cu") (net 17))
 (segment (start 186.4883 68.0983) (end 186.5 68.11) (width 0.2) (layer "F.Cu") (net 17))
 (segment (start 151.3293 60.8293) (end 151.5 61) (width 0.2) (layer "F.Cu") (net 17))
 (segment (start 186.5 68.11) (end 191.11 68.11) (width 0.2) (layer "F.Cu") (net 17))
 (segment (start 134.425 58.5017) (end 135.5767 58.5017) (width 0.2) (layer "F.Cu") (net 17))
 (segment (start 174.5 61) (end 181.5 68) (width 0.2) (layer "F.Cu") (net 17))
 (segment (start 191.11 68.11) (end 191.63 68.63) (width 0.2) (layer "F.Cu") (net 17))
 (segment (start 134.425 57.35) (end 134.425 58.5017) (width 0.2) (layer "F.Cu") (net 17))
 (segment (start 198.8046 95.6546) (end 136.8932 95.6546) (width 0.2) (layer "F.Cu") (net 30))
 (segment (start 201.79 98.64) (end 198.8046 95.6546) (width 0.2) (layer "F.Cu") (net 30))
 (segment (start 136.8932 95.6546) (end 134.3976 93.159) (width 0.2) (layer "F.Cu") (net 30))
 (via (at 134.3976 93.159) (size 0.6) (drill 0.3) (layers "F.Cu" "B.Cu") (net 30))
 (segment (start 133.9733 56.0017) (end 134.425 56.0017) (width 0.2) (layer "B.Cu") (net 30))
 (segment (start 133.1313 91.8927) (end 133.1313 56.8437) (width 0.2) (layer "B.Cu") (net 30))
 (segment (start 134.3976 93.159) (end 133.1313 91.8927) (width 0.2) (layer "B.Cu") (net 30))
 (segment (start 133.1313 56.8437) (end 133.9733 56.0017) (width 0.2) (layer "B.Cu") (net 30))
 (segment (start 134.425 54.85) (end 134.425 56.0017) (width 0.2) (layer "B.Cu") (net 30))
 (segment (start 134.425 53.5017) (end 168.1435 53.5017) (width 0.2) (layer "F.Cu") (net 16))
 (segment (start 194.17 67.67) (end 194.17 73.24) (width 0.2) (layer "F.Cu") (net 16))
 (segment (start 187.1418 66.5) (end 193 66.5) (width 0.2) (layer "F.Cu") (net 16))
 (segment (start 181 66.3582) (end 187 66.3582) (width 0.2) (layer "F.Cu") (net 16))
 (segment (start 134.425 52.35) (end 134.425 53.5017) (width 0.2) (layer "F.Cu") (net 16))
 (segment (start 187 66.3582) (end 187.1418 66.5) (width 0.2) (layer "F.Cu") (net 16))
 (segment (start 168.1435 53.5017) (end 181 66.3582) (width 0.2) (layer "F.Cu") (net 16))
 (segment (start 193 66.5) (end 194.17 67.67) (width 0.2) (layer "F.Cu") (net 16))
 (segment (start 135.2168 92.3287) (end 134.3771 92.3287) (width 0.2) (layer "F.Cu") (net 26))
 (segment (start 189.0936 96.1036) (end 191.63 98.64) (width 0.2) (layer "F.Cu") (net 26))
 (segment (start 136.4914 96.1036) (end 189.0936 96.1036) (width 0.2) (layer "F.Cu") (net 26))
 (segment (start 134.3771 92.3287) (end 133.7959 92.9099) (width 0.2) (layer "F.Cu") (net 26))
 (segment (start 133.7959 93.4081) (end 136.4914 96.1036) (width 0.2) (layer "F.Cu") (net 26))
 (segment (start 133.7959 92.9099) (end 133.7959 93.4081) (width 0.2) (layer "F.Cu") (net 26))
 (via (at 135.2168 92.3287) (size 0.6) (drill 0.3) (layers "F.Cu" "B.Cu") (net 26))
 (segment (start 134.425 62.35) (end 135.7489 63.6739) (width 0.2) (layer "B.Cu") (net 26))
 (segment (start 135.7489 91.7966) (end 135.2168 92.3287) (width 0.2) (layer "B.Cu") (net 26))
 (segment (start 135.7489 63.6739) (end 135.7489 91.7966) (width 0.2) (layer "B.Cu") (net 26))
 (segment (start 151.7627 51.4992) (end 154.3119 48.95) (width 0.2) (layer "F.Cu") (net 6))
 (segment (start 188.95 48.95) (end 193 48.95) (width 0.2) (layer "F.Cu") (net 6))
 (segment (start 189.125 47.9) (end 189.125 46) (width 0.2) (layer "F.Cu") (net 6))
 (segment (start 154.3119 48.95) (end 188.95 48.95) (width 0.2) (layer "F.Cu") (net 6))
 (via (at 151.7627 51.4992) (size 0.6) (drill 0.3) (layers "F.Cu" "B.Cu") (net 6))
 (segment (start 143.75 86.15) (end 145.7717 86.15) (width 0.2) (layer "B.Cu") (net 6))
 (segment (start 151.7627 80.159) (end 151.7627 51.4992) (width 0.2) (layer "B.Cu") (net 6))
 (segment (start 145.7717 86.15) (end 151.7627 80.159) (width 0.2) (layer "B.Cu") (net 6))
 (segment (start 211.3685 76.3615) (end 214.49 73.24) (width 0.2) (layer "F.Cu") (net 7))
 (segment (start 134.425 78.9983) (end 136.1446 78.9983) (width 0.2) (layer "F.Cu") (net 7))
 (segment (start 136.1446 78.9983) (end 138.7814 76.3615) (width 0.2) (layer "F.Cu") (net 7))
 (segment (start 138.7814 76.3615) (end 211.3685 76.3615) (width 0.2) (layer "F.Cu") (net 7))
 (segment (start 134.425 80.15) (end 134.425 78.9983) (width 0.2) (layer "F.Cu") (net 7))
 (segment (start 189 71) (end 187.5 69.5) (width 0.2) (layer "F.Cu") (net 8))
 (segment (start 187.5 69.5) (end 176.5 69.5) (width 0.2) (layer "F.Cu") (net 8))
 (segment (start 137.6557 74.4193) (end 135.5767 76.4983) (width 0.2) (layer "F.Cu") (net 8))
 (segment (start 155 57.5) (end 151.55 57.5) (width 0.2) (layer "F.Cu") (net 8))
 (segment (start 134.425 77.65) (end 134.425 76.4983) (width 0.2) (layer "F.Cu") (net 8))
 (segment (start 146.9788 74.4193) (end 137.6557 74.4193) (width 0.2) (layer "F.Cu") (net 8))
 (segment (start 176.5 69.5) (end 172 65) (width 0.2) (layer "F.Cu") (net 8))
 (segment (start 189 73.15) (end 189 71) (width 0.2) (layer "F.Cu") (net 8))
 (segment (start 151.55 57.5) (end 148.725 54.675) (width 0.2) (layer "F.Cu") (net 8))
 (segment (start 172 65) (end 157.5 65) (width 0.2) (layer "F.Cu") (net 8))
 (segment (start 135.5767 76.4983) (end 134.425 76.4983) (width 0.2) (layer "F.Cu") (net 8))
 (segment (start 189.09 73.24) (end 189 73.15) (width 0.2) (layer "F.Cu") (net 8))
 (via (at 157.5 65) (size 0.6) (drill 0.3) (layers "F.Cu" "B.Cu") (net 8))
 (via (at 146.9788 74.4193) (size 0.6) (drill 0.3) (layers "F.Cu" "B.Cu") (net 8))
 (via (at 155 57.5) (size 0.6) (drill 0.3) (layers "F.Cu" "B.Cu") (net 8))
 (segment (start 148.2931 55.8267) (end 146.8434 57.2764) (width 0.2) (layer "B.Cu") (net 8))
 (segment (start 146.8434 57.2764) (end 146.8434 74.2839) (width 0.2) (layer "B.Cu") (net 8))
 (segment (start 146.8434 74.2839) (end 146.9788 74.4193) (width 0.2) (layer "B.Cu") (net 8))
 (segment (start 157.5 60) (end 155 57.5) (width 0.2) (layer "B.Cu") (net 8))
 (segment (start 157.5 65) (end 157.5 60) (width 0.2) (layer "B.Cu") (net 8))
 (segment (start 148.725 54.675) (end 148.725 55.8267) (width 0.2) (layer "B.Cu") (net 8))
 (segment (start 148.725 55.8267) (end 148.2931 55.8267) (width 0.2) (layer "B.Cu") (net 8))
 (segment (start 179 70.5) (end 176 70.5) (width 0.2) (layer "F.Cu") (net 9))
 (segment (start 134.425 75.15) (end 134.425 73.9983) (width 0.2) (layer "F.Cu") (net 9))
 (segment (start 181.47 72.97) (end 179 70.5) (width 0.2) (layer "F.Cu") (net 9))
 (segment (start 145.105 73.9983) (end 147.4451 71.6582) (width 0.2) (layer "F.Cu") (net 9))
 (segment (start 172 66.5) (end 156.5 66.5) (width 0.2) (layer "F.Cu") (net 9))
 (segment (start 176 70.5) (end 172 66.5) (width 0.2) (layer "F.Cu") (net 9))
 (segment (start 181.47 73.24) (end 181.47 72.97) (width 0.2) (layer "F.Cu") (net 9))
 (segment (start 156.5 66.5) (end 156 67) (width 0.2) (layer "F.Cu") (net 9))
 (segment (start 134.425 73.9983) (end 145.105 73.9983) (width 0.2) (layer "F.Cu") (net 9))
 (segment (start 149.6033 69.5) (end 147.4451 71.6582) (width 0.2) (layer "F.Cu") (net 9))
 (segment (start 153 69.5) (end 149.6033 69.5) (width 0.2) (layer "F.Cu") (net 9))
 (via (at 147.4451 71.6582) (size 0.6) (drill 0.3) (layers "F.Cu" "B.Cu") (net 9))
 (via (at 153 69.5) (size 0.6) (drill 0.3) (layers "F.Cu" "B.Cu") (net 9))
 (via (at 156 67) (size 0.6) (drill 0.3) (layers "F.Cu" "B.Cu") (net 9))
 (segment (start 148.2733 58.3267) (end 148.725 58.3267) (width 0.2) (layer "B.Cu") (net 9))
 (segment (start 147.4451 71.6582) (end 147.4451 59.1549) (width 0.2) (layer "B.Cu") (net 9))
 (segment (start 148.725 57.175) (end 148.725 58.3267) (width 0.2) (layer "B.Cu") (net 9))
 (segment (start 156 67) (end 155.5 67) (width 0.2) (layer "B.Cu") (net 9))
 (segment (start 147.4451 59.1549) (end 148.2733 58.3267) (width 0.2) (layer "B.Cu") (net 9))
 (segment (start 155.5 67) (end 153 69.5) (width 0.2) (layer "B.Cu") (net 9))
 (segment (start 205.9247 45.4247) (end 195.5967 45.4247) (width 0.2) (layer "F.Cu") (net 5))
 (segment (start 194.2062 46.8152) (end 190.8314 46.8152) (width 0.2) (layer "F.Cu") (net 5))
 (segment (start 190.8314 46.8152) (end 190.4134 46.3972) (width 0.2) (layer "F.Cu") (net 5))
 (segment (start 207.5 47) (end 205.9247 45.4247) (width 0.2) (layer "F.Cu") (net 5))
 (segment (start 195.5967 45.4247) (end 194.2062 46.8152) (width 0.2) (layer "F.Cu") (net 5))
 (segment (start 177.675 51.85) (end 178.775 52.95) (width 0.2) (layer "F.Cu") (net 2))
 (segment (start 178.775 52.95) (end 182.175 52.95) (width 0.2) (layer "F.Cu") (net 2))
 (segment (start 182.175 52.95) (end 187.125 52.95) (width 0.2) (layer "F.Cu") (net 2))
 (segment (start 182.175 55.05) (end 182.175 52.95) (width 0.2) (layer "F.Cu") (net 2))
 (segment (start 173.2404 98.8699) (end 172.8615 98.491) (width 0.2) (layer "F.Cu") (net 28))
 (segment (start 172.8615 98.491) (end 173.2404 98.8699) (width 0.2) (layer "F.Cu") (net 28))
 (segment (start 173.9532 56) (end 173.4433 56.5099) (width 0.2) (layer "F.Cu") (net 28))
 (segment (start 174.5937 100.2232) (end 172.8615 98.491) (width 0.2) (layer "F.Cu") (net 28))
 (segment (start 195.1268 100.2232) (end 174.5937 100.2232) (width 0.2) (layer "F.Cu") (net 28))
 (segment (start 177.5 56) (end 173.9532 56) (width 0.2) (layer "F.Cu") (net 28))
 (segment (start 196.71 98.64) (end 195.1268 100.2232) (width 0.2) (layer "F.Cu") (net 28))
 (via (at 173.4433 56.5099) (size 0.6) (drill 0.3) (layers "F.Cu" "B.Cu") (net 28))
 (via (at 172.8615 98.491) (size 0.6) (drill 0.3) (layers "F.Cu" "B.Cu") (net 28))
 (segment (start 172.8615 98.491) (end 172.8615 57.0917) (width 0.2) (layer "B.Cu") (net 28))
 (segment (start 172.8615 57.0917) (end 173.4433 56.5099) (width 0.2) (layer "B.Cu") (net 28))
 (segment (start 202.9495 68.4495) (end 199.4 64.9) (width 0.2) (layer "F.Cu") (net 34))
 (segment (start 214.6103 68.4495) (end 202.9495 68.4495) (width 0.2) (layer "F.Cu") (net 34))
 (via (at 214.6103 68.4495) (size 0.6) (drill 0.3) (layers "F.Cu" "B.Cu") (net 34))
 (segment (start 218.6957 94.4343) (end 218.6957 72.5349) (width 0.2) (layer "B.Cu") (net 34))
 (segment (start 214.49 98.64) (end 218.6957 94.4343) (width 0.2) (layer "B.Cu") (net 34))
 (segment (start 218.6957 72.5349) (end 214.6103 68.4495) (width 0.2) (layer "B.Cu") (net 34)))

